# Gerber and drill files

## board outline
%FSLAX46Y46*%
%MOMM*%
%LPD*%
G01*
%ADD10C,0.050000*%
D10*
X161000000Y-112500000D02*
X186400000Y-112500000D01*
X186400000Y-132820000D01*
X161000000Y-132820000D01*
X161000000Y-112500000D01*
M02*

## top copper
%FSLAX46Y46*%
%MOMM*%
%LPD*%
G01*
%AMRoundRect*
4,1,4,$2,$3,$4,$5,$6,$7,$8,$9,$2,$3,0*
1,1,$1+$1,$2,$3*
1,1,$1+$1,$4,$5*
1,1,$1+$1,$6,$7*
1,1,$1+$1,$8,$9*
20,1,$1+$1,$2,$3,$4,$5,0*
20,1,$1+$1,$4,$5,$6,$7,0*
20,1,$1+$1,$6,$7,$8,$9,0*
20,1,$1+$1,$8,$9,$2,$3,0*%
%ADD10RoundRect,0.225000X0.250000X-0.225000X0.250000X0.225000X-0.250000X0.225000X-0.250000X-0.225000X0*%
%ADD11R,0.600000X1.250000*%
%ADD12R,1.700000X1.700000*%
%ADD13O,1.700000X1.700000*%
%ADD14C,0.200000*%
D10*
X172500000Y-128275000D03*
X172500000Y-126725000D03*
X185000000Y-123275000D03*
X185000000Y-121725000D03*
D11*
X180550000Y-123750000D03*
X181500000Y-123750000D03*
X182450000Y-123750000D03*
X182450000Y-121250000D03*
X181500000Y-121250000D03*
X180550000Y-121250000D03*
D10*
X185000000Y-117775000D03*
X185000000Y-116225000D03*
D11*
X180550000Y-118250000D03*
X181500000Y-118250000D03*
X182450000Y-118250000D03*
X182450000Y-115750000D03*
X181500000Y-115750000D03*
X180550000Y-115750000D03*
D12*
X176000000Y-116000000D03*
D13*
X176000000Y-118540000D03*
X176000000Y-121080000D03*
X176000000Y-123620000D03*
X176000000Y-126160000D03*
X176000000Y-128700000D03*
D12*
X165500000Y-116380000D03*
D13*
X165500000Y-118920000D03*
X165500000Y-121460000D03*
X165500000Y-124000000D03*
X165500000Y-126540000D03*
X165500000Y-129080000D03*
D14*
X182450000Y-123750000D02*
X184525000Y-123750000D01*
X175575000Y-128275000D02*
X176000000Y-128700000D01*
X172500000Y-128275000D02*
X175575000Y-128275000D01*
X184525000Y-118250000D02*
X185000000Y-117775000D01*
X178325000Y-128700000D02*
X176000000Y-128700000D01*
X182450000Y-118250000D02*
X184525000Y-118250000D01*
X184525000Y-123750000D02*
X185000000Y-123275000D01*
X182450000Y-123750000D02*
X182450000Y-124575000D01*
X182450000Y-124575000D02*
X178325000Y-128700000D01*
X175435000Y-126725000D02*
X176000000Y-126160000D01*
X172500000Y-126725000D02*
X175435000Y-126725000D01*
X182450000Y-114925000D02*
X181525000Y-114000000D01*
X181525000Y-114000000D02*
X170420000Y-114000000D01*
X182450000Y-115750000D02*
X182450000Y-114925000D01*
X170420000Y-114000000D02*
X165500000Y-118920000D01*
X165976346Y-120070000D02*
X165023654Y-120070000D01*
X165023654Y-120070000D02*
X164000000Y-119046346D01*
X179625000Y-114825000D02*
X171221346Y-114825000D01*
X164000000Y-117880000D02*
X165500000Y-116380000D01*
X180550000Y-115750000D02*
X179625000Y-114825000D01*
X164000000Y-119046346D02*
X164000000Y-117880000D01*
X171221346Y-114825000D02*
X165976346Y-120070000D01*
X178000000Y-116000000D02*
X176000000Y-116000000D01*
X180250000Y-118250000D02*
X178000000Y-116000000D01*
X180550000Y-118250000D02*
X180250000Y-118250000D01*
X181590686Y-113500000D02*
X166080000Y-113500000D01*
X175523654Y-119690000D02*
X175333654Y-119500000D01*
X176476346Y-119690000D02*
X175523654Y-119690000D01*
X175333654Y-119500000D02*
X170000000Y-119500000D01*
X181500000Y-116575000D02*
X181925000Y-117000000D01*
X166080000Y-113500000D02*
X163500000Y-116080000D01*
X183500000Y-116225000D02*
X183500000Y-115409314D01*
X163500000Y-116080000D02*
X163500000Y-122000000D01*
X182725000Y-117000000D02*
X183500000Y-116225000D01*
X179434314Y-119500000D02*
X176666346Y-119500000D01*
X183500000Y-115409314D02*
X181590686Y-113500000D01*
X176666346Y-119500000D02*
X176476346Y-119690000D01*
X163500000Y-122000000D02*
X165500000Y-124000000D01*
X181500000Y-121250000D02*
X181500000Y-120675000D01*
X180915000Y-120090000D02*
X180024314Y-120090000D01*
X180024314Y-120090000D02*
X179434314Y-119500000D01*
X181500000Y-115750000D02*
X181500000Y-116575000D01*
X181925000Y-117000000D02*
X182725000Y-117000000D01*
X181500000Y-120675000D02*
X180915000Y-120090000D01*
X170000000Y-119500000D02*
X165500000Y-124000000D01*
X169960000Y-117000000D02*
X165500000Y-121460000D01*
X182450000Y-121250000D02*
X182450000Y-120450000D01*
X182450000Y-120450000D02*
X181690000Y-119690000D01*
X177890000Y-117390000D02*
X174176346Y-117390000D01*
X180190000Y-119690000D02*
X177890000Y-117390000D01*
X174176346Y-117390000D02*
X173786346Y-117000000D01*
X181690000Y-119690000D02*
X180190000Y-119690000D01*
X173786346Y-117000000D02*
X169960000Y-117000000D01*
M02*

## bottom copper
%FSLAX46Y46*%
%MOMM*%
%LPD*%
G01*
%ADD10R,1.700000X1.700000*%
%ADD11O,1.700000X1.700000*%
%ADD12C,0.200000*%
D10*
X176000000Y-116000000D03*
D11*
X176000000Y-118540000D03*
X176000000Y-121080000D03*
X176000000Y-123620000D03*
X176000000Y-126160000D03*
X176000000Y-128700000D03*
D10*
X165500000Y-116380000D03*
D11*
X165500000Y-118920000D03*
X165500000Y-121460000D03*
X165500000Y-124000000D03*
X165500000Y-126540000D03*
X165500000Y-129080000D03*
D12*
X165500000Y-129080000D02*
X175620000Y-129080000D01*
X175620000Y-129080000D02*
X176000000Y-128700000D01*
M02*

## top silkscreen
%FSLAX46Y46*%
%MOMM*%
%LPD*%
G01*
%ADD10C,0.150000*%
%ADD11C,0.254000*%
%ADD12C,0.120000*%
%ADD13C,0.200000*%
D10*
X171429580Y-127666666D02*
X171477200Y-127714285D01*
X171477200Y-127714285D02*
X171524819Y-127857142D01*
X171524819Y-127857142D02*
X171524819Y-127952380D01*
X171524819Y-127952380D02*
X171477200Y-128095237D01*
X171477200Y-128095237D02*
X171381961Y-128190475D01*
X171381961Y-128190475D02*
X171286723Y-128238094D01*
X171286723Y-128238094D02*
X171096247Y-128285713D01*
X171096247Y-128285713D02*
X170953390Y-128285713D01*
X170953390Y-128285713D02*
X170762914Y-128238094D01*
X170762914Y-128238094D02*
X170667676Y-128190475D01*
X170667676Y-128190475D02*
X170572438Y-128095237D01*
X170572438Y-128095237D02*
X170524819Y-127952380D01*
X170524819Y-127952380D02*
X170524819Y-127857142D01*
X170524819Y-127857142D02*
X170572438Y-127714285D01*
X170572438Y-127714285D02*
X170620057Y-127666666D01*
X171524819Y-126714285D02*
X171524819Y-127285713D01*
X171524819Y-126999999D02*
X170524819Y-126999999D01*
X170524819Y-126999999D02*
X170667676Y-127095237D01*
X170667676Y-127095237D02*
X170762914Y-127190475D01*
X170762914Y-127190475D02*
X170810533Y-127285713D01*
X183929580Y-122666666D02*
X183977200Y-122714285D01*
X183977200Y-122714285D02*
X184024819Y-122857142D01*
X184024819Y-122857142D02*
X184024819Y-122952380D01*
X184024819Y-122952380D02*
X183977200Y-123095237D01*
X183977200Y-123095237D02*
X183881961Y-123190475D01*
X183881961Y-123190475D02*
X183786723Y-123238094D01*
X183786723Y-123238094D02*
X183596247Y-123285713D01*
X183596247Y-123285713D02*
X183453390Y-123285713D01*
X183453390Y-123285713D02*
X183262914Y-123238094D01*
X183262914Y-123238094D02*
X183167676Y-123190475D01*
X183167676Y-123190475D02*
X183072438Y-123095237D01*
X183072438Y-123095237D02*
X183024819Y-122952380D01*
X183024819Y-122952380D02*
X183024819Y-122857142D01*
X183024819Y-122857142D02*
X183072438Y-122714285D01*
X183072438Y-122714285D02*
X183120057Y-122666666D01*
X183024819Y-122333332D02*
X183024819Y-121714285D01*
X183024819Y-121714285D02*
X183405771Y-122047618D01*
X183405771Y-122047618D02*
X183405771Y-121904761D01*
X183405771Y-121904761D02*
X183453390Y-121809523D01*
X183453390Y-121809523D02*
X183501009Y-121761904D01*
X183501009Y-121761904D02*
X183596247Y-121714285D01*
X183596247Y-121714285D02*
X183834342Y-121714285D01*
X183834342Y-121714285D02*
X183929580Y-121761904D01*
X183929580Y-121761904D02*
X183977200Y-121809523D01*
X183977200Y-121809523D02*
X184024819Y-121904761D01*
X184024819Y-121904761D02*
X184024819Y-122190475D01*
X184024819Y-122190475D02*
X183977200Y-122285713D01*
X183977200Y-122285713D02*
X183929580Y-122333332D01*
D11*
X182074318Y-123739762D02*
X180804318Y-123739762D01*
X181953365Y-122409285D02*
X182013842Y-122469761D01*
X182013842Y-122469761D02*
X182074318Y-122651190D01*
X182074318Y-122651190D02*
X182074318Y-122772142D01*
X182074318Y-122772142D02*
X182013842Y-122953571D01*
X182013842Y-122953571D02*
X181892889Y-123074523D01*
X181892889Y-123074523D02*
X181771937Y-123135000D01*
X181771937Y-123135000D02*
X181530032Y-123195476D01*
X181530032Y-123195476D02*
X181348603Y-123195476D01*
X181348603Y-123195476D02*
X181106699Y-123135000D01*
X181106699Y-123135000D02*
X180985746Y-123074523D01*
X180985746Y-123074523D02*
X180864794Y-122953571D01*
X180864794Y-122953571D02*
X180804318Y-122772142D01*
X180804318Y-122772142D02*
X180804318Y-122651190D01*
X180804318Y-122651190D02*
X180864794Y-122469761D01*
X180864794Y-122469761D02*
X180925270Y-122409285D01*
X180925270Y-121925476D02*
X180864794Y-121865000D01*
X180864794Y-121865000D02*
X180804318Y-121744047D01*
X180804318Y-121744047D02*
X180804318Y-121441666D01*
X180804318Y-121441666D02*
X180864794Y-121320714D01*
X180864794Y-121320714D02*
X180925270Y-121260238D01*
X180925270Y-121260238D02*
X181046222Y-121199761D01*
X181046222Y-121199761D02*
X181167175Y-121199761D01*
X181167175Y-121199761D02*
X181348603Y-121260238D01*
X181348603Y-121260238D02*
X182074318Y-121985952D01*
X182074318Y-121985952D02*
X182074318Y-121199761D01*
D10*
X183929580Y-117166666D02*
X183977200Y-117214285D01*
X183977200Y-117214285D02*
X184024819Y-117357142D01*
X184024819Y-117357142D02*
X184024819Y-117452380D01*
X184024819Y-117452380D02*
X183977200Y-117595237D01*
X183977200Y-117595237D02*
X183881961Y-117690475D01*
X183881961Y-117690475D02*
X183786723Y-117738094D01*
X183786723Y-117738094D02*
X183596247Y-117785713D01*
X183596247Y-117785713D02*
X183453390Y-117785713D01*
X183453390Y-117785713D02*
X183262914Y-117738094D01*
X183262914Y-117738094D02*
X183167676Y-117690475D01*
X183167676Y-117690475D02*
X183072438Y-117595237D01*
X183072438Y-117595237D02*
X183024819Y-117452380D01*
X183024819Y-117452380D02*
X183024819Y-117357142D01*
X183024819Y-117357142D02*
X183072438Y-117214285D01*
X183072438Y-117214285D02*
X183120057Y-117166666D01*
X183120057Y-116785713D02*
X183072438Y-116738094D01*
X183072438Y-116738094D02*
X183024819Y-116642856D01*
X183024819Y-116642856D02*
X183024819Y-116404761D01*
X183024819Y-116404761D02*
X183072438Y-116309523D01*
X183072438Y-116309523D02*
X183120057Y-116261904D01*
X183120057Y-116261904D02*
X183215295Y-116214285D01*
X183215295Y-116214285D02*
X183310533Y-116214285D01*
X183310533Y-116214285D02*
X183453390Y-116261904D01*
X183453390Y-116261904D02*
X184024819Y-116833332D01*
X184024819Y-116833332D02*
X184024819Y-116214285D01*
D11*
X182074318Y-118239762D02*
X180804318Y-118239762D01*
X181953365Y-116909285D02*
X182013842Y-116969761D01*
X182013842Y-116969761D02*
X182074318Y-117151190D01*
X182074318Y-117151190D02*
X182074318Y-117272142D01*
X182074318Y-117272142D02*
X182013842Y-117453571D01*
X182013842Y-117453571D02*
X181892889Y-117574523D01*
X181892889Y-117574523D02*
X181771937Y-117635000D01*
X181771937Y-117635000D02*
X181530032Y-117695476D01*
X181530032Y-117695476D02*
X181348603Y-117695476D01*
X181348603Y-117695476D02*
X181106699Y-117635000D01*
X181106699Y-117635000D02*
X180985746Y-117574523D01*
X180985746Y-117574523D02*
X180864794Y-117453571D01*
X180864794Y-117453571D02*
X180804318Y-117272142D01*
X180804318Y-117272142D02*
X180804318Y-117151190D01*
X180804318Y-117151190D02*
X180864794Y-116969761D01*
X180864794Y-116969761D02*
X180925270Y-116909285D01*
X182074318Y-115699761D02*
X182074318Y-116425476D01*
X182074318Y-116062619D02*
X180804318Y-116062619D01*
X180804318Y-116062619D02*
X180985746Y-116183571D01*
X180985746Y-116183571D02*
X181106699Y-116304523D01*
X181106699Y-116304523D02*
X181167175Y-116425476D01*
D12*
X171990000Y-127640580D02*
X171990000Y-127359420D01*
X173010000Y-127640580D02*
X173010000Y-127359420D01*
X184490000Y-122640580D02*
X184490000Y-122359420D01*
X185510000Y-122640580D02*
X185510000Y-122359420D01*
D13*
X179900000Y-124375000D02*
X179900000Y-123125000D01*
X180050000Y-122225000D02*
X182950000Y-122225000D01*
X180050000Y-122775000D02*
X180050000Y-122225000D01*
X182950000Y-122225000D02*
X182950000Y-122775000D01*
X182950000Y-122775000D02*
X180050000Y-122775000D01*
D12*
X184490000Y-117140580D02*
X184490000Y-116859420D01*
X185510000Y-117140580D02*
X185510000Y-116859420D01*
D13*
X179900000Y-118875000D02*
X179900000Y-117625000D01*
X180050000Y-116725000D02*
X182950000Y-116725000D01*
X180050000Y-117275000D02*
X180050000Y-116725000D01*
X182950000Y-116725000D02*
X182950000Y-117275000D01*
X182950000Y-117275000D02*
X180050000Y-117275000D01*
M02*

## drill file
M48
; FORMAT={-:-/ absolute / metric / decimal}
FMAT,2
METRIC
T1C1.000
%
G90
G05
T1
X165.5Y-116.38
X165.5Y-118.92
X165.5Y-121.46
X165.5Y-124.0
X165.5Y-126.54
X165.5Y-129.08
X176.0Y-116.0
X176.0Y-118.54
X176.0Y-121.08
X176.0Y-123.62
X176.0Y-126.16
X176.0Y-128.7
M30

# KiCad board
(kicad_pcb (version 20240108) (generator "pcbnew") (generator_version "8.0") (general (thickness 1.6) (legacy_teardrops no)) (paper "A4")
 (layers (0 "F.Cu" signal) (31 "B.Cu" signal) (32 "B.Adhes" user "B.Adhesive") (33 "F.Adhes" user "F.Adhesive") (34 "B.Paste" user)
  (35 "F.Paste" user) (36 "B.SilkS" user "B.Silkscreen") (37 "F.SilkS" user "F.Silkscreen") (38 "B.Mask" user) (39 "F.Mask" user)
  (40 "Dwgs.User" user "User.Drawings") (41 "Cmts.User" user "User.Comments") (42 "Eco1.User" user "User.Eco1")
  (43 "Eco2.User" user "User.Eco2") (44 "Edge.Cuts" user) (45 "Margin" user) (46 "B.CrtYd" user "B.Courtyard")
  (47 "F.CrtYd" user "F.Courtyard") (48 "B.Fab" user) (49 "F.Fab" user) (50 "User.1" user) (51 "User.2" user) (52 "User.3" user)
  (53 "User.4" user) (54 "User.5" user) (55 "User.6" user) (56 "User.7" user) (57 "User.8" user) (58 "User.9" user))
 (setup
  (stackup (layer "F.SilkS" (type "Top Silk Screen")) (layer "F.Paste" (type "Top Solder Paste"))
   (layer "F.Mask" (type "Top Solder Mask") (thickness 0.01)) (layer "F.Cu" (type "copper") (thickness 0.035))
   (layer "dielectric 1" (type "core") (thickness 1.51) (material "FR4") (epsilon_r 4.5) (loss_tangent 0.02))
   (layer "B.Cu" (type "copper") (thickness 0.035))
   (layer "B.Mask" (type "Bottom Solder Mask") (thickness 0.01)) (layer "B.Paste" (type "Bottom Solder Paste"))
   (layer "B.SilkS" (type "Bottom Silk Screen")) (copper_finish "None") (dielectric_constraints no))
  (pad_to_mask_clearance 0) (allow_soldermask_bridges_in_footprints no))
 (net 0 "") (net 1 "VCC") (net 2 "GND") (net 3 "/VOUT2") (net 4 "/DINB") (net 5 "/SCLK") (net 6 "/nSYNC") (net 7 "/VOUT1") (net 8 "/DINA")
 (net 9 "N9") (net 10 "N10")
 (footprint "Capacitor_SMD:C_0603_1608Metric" (layer "F.Cu") (at 172.5 127.5 90)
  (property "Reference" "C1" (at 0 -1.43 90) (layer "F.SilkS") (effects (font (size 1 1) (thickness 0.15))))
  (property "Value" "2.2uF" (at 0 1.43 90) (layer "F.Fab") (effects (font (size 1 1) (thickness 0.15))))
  (fp_line (start -0.14058 -0.51) (end 0.14058 -0.51) (stroke (width 0.12) (type solid)) (layer "F.SilkS"))
  (fp_line (start -0.14058 0.51) (end 0.14058 0.51) (stroke (width 0.12) (type solid)) (layer "F.SilkS"))
  (pad "1" smd roundrect (at -0.775 0 90) (size 0.9 0.95) (layers "F.Cu" "F.Paste" "F.Mask") (roundrect_rratio 0.25) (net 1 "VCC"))
  (pad "2" smd roundrect (at 0.775 0 90) (size 0.9 0.95) (layers "F.Cu" "F.Paste" "F.Mask") (roundrect_rratio 0.25) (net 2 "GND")))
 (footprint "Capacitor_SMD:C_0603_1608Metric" (layer "F.Cu") (at 185 122.5 90)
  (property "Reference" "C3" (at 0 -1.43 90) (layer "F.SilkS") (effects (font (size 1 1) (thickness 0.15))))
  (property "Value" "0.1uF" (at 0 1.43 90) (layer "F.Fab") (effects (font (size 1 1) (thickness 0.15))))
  (fp_line (start -0.14058 -0.51) (end 0.14058 -0.51) (stroke (width 0.12) (type solid)) (layer "F.SilkS"))
  (fp_line (start -0.14058 0.51) (end 0.14058 0.51) (stroke (width 0.12) (type solid)) (layer "F.SilkS"))
  (pad "1" smd roundrect (at -0.775 0 90) (size 0.9 0.95) (layers "F.Cu" "F.Paste" "F.Mask") (roundrect_rratio 0.25) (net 1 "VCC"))
  (pad "2" smd roundrect (at 0.775 0 90) (size 0.9 0.95) (layers "F.Cu" "F.Paste" "F.Mask") (roundrect_rratio 0.25) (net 2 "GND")))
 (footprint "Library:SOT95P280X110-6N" (layer "F.Cu") (at 181.5 122.5 90)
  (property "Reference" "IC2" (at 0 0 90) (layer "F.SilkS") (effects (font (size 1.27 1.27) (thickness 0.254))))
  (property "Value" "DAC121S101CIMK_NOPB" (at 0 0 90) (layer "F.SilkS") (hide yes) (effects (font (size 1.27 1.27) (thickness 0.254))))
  (fp_line (start -1.875 -1.6) (end -0.625 -1.6) (stroke (width 0.2) (type solid)) (layer "F.SilkS"))
  (fp_line (start 0.275 -1.45) (end 0.275 1.45) (stroke (width 0.2) (type solid)) (layer "F.SilkS"))
  (fp_line (start -0.275 -1.45) (end 0.275 -1.45) (stroke (width 0.2) (type solid)) (layer "F.SilkS"))
  (fp_line (start 0.275 1.45) (end -0.275 1.45) (stroke (width 0.2) (type solid)) (layer "F.SilkS"))
  (fp_line (start -0.275 1.45) (end -0.275 -1.45) (stroke (width 0.2) (type solid)) (layer "F.SilkS"))
  (pad "1" smd rect (at -1.25 -0.95 180) (size 0.6 1.25) (layers "F.Cu" "F.Paste" "F.Mask") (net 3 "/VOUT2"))
  (pad "2" smd rect (at -1.25 0 180) (size 0.6 1.25) (layers "F.Cu" "F.Paste" "F.Mask") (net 2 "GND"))
  (pad "3" smd rect (at -1.25 0.95 180) (size 0.6 1.25) (layers "F.Cu" "F.Paste" "F.Mask") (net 1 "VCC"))
  (pad "4" smd rect (at 1.25 0.95 180) (size 0.6 1.25) (layers "F.Cu" "F.Paste" "F.Mask") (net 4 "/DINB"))
  (pad "5" smd rect (at 1.25 0 180) (size 0.6 1.25) (layers "F.Cu" "F.Paste" "F.Mask") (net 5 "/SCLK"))
  (pad "6" smd rect (at 1.25 -0.95 180) (size 0.6 1.25) (layers "F.Cu" "F.Paste" "F.Mask") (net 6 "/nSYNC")))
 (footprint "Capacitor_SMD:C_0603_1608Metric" (layer "F.Cu") (at 185 117 90)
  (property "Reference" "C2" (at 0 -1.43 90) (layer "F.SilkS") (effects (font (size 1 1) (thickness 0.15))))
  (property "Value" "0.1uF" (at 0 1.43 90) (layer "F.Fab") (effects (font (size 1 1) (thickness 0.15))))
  (fp_line (start -0.14058 -0.51) (end 0.14058 -0.51) (stroke (width 0.12) (type solid)) (layer "F.SilkS"))
  (fp_line (start -0.14058 0.51) (end 0.14058 0.51) (stroke (width 0.12) (type solid)) (layer "F.SilkS"))
  (pad "1" smd roundrect (at -0.775 0 90) (size 0.9 0.95) (layers "F.Cu" "F.Paste" "F.Mask") (roundrect_rratio 0.25) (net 1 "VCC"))
  (pad "2" smd roundrect (at 0.775 0 90) (size 0.9 0.95) (layers "F.Cu" "F.Paste" "F.Mask") (roundrect_rratio 0.25) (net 2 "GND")))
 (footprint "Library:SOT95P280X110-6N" (layer "F.Cu") (at 181.5 117 90)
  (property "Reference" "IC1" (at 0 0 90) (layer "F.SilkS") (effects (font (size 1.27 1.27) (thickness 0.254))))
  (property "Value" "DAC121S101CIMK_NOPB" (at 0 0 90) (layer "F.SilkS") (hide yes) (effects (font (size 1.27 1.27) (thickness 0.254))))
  (fp_line (start -1.875 -1.6) (end -0.625 -1.6) (stroke (width 0.2) (type solid)) (layer "F.SilkS"))
  (fp_line (start 0.275 -1.45) (end 0.275 1.45) (stroke (width 0.2) (type solid)) (layer "F.SilkS"))
  (fp_line (start -0.275 -1.45) (end 0.275 -1.45) (stroke (width 0.2) (type solid)) (layer "F.SilkS"))
  (fp_line (start 0.275 1.45) (end -0.275 1.45) (stroke (width 0.2) (type solid)) (layer "F.SilkS"))
  (fp_line (start -0.275 1.45) (end -0.275 -1.45) (stroke (width 0.2) (type solid)) (layer "F.SilkS"))
  (pad "1" smd rect (at -1.25 -0.95 180) (size 0.6 1.25) (layers "F.Cu" "F.Paste" "F.Mask") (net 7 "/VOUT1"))
  (pad "2" smd rect (at -1.25 0 180) (size 0.6 1.25) (layers "F.Cu" "F.Paste" "F.Mask") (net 2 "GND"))
  (pad "3" smd rect (at -1.25 0.95 180) (size 0.6 1.25) (layers "F.Cu" "F.Paste" "F.Mask") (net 1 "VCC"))
  (pad "4" smd rect (at 1.25 0.95 180) (size 0.6 1.25) (layers "F.Cu" "F.Paste" "F.Mask") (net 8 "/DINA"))
  (pad "5" smd rect (at 1.25 0 180) (size 0.6 1.25) (layers "F.Cu" "F.Paste" "F.Mask") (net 5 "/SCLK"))
  (pad "6" smd rect (at 1.25 -0.95 180) (size 0.6 1.25) (layers "F.Cu" "F.Paste" "F.Mask") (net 6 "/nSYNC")))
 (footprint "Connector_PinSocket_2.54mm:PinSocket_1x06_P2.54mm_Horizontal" (layer "B.Cu") (at 176 116 180)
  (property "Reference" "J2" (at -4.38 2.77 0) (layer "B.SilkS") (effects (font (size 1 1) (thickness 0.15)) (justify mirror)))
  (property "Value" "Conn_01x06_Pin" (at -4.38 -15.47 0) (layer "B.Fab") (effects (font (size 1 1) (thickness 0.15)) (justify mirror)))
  (pad "1" thru_hole rect (at 0 0 180) (size 1.7 1.7) (drill 1) (layers "*.Cu" "*.Mask") (remove_unused_layers no) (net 7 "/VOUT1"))
  (pad "2" thru_hole oval (at 0 -2.54 180) (size 1.7 1.7) (drill 1) (layers "*.Cu" "*.Mask") (remove_unused_layers no) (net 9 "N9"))
  (pad "3" thru_hole oval (at 0 -5.08 180) (size 1.7 1.7) (drill 1) (layers "*.Cu" "*.Mask") (remove_unused_layers no) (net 3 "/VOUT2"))
  (pad "4" thru_hole oval (at 0 -7.62 180) (size 1.7 1.7) (drill 1) (layers "*.Cu" "*.Mask") (remove_unused_layers no) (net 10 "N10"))
  (pad "5" thru_hole oval (at 0 -10.16 180) (size 1.7 1.7) (drill 1) (layers "*.Cu" "*.Mask") (remove_unused_layers no) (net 2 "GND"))
  (pad "6" thru_hole oval (at 0 -12.7 180) (size 1.7 1.7) (drill 1) (layers "*.Cu" "*.Mask") (remove_unused_layers no) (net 1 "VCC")))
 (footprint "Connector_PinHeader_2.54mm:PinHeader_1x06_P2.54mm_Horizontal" (layer "B.Cu") (at 165.5 116.38 180)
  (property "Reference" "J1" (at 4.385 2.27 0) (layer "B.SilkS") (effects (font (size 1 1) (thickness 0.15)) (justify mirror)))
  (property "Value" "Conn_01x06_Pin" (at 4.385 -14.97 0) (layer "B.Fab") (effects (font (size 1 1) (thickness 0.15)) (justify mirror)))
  (pad "1" thru_hole rect (at 0 0 180) (size 1.7 1.7) (drill 1) (layers "*.Cu" "*.Mask") (remove_unused_layers no) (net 6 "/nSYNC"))
  (pad "2" thru_hole oval (at 0 -2.54 180) (size 1.7 1.7) (drill 1) (layers "*.Cu" "*.Mask") (remove_unused_layers no) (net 8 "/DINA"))
  (pad "3" thru_hole oval (at 0 -5.08 180) (size 1.7 1.7) (drill 1) (layers "*.Cu" "*.Mask") (remove_unused_layers no) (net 4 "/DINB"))
  (pad "4" thru_hole oval (at 0 -7.62 180) (size 1.7 1.7) (drill 1) (layers "*.Cu" "*.Mask") (remove_unused_layers no) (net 5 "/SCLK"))
  (pad "5" thru_hole oval (at 0 -10.16 180) (size 1.7 1.7) (drill 1) (layers "*.Cu" "*.Mask") (remove_unused_layers no) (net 2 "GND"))
  (pad "6" thru_hole oval (at 0 -12.7 180) (size 1.7 1.7) (drill 1) (layers "*.Cu" "*.Mask") (remove_unused_layers no) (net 1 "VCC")))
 (gr_rect (start 161 112.5) (end 186.4 132.82) (stroke (width 0.05) (type default)) (fill none) (layer "Edge.Cuts"))
 (segment (start 182.45 123.75) (end 184.525 123.75) (width 0.2) (layer "F.Cu") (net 1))
 (segment (start 175.575 128.275) (end 176 128.7) (width 0.2) (layer "F.Cu") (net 1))
 (segment (start 172.5 128.275) (end 175.575 128.275) (width 0.2) (layer "F.Cu") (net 1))
 (segment (start 184.525 118.25) (end 185 117.775) (width 0.2) (layer "F.Cu") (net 1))
 (segment (start 178.325 128.7) (end 176 128.7) (width 0.2) (layer "F.Cu") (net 1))
 (segment (start 182.45 118.25) (end 184.525 118.25) (width 0.2) (layer "F.Cu") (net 1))
 (segment (start 184.525 123.75) (end 185 123.275) (width 0.2) (layer "F.Cu") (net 1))
 (segment (start 182.45 123.75) (end 182.45 124.575) (width 0.2) (layer "F.Cu") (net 1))
 (segment (start 182.45 124.575) (end 178.325 128.7) (width 0.2) (layer "F.Cu") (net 1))
 (segment (start 165.5 129.08) (end 175.62 129.08) (width 0.2) (layer "B.Cu") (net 1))
 (segment (start 175.62 129.08) (end 176 128.7) (width 0.2) (layer "B.Cu") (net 1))
 (segment (start 175.435 126.725) (end 176 126.16) (width 0.2) (layer "F.Cu") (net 2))
 (segment (start 172.5 126.725) (end 175.435 126.725) (width 0.2) (layer "F.Cu") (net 2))
 (segment (start 182.45 114.925) (end 181.525 114) (width 0.2) (layer "F.Cu") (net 8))
 (segment (start 181.525 114) (end 170.42 114) (width 0.2) (layer "F.Cu") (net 8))
 (segment (start 182.45 115.75) (end 182.45 114.925) (width 0.2) (layer "F.Cu") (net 8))
 (segment (start 170.42 114) (end 165.5 118.92) (width 0.2) (layer "F.Cu") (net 8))
 (segment (start 165.976346 120.07) (end 165.023654 120.07) (width 0.2) (layer "F.Cu") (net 6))
 (segment (start 165.023654 120.07) (end 164 119.046346) (width 0.2) (layer "F.Cu") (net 6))
 (segment (start 179.625 114.825) (end 171.221346 114.825) (width 0.2) (layer "F.Cu") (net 6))
 (segment (start 164 117.88) (end 165.5 116.38) (width 0.2) (layer "F.Cu") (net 6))
 (segment (start 180.55 115.75) (end 179.625 114.825) (width 0.2) (layer "F.Cu") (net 6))
 (segment (start 164 119.046346) (end 164 117.88) (width 0.2) (layer "F.Cu") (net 6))
 (segment (start 171.221346 114.825) (end 165.976346 120.07) (width 0.2) (layer "F.Cu") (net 6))
 (segment (start 178 116) (end 176 116) (width 0.2) (layer "F.Cu") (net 7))
 (segment (start 180.25 118.25) (end 178 116) (width 0.2) (layer "F.Cu") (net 7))
 (segment (start 180.55 118.25) (end 180.25 118.25) (width 0.2) (layer "F.Cu") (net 7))
 (segment (start 181.590686 113.5) (end 166.08 113.5) (width 0.2) (layer "F.Cu") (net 5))
 (segment (start 175.523654 119.69) (end 175.333654 119.5) (width 0.2) (layer "F.Cu") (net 5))
 (segment (start 176.476346 119.69) (end 175.523654 119.69) (width 0.2) (layer "F.Cu") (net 5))
 (segment (start 175.333654 119.5) (end 170 119.5) (width 0.2) (layer "F.Cu") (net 5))
 (segment (start 181.5 116.575) (end 181.925 117) (width 0.2) (layer "F.Cu") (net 5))
 (segment (start 166.08 113.5) (end 163.5 116.08) (width 0.2) (layer "F.Cu") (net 5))
 (segment (start 183.5 116.225) (end 183.5 115.409314) (width 0.2) (layer "F.Cu") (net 5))
 (segment (start 163.5 116.08) (end 163.5 122) (width 0.2) (layer "F.Cu") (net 5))
 (segment (start 182.725 117) (end 183.5 116.225) (width 0.2) (layer "F.Cu") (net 5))
 (segment (start 179.434314 119.5) (end 176.666346 119.5) (width 0.2) (layer "F.Cu") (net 5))
 (segment (start 183.5 115.409314) (end 181.590686 113.5) (width 0.2) (layer "F.Cu") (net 5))
 (segment (start 176.666346 119.5) (end 176.476346 119.69) (width 0.2) (layer "F.Cu") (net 5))
 (segment (start 163.5 122) (end 165.5 124) (width 0.2) (layer "F.Cu") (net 5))
 (segment (start 181.5 121.25) (end 181.5 120.675) (width 0.2) (layer "F.Cu") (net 5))
 (segment (start 180.915 120.09) (end 180.024314 120.09) (width 0.2) (layer "F.Cu") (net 5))
 (segment (start 180.024314 120.09) (end 179.434314 119.5) (width 0.2) (layer "F.Cu") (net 5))
 (segment (start 181.5 115.75) (end 181.5 116.575) (width 0.2) (layer "F.Cu") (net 5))
 (segment (start 181.925 117) (end 182.725 117) (width 0.2) (layer "F.Cu") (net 5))
 (segment (start 181.5 120.675) (end 180.915 120.09) (width 0.2) (layer "F.Cu") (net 5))
 (segment (start 170 119.5) (end 165.5 124) (width 0.2) (layer "F.Cu") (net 5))
 (segment (start 169.96 117) (end 165.5 121.46) (width 0.2) (layer "F.Cu") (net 4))
 (segment (start 182.45 121.25) (end 182.45 120.45) (width 0.2) (layer "F.Cu") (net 4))
 (segment (start 182.45 120.45) (end 181.69 119.69) (width 0.2) (layer "F.Cu") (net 4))
 (segment (start 177.89 117.39) (end 174.176346 117.39) (width 0.2) (layer "F.Cu") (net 4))
 (segment (start 180.19 119.69) (end 177.89 117.39) (width 0.2) (layer "F.Cu") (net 4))
 (segment (start 174.176346 117.39) (end 173.786346 117) (width 0.2) (layer "F.Cu") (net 4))
 (segment (start 181.69 119.69) (end 180.19 119.69) (width 0.2) (layer "F.Cu") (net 4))
 (segment (start 173.786346 117) (end 169.96 117) (width 0.2) (layer "F.Cu") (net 4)))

